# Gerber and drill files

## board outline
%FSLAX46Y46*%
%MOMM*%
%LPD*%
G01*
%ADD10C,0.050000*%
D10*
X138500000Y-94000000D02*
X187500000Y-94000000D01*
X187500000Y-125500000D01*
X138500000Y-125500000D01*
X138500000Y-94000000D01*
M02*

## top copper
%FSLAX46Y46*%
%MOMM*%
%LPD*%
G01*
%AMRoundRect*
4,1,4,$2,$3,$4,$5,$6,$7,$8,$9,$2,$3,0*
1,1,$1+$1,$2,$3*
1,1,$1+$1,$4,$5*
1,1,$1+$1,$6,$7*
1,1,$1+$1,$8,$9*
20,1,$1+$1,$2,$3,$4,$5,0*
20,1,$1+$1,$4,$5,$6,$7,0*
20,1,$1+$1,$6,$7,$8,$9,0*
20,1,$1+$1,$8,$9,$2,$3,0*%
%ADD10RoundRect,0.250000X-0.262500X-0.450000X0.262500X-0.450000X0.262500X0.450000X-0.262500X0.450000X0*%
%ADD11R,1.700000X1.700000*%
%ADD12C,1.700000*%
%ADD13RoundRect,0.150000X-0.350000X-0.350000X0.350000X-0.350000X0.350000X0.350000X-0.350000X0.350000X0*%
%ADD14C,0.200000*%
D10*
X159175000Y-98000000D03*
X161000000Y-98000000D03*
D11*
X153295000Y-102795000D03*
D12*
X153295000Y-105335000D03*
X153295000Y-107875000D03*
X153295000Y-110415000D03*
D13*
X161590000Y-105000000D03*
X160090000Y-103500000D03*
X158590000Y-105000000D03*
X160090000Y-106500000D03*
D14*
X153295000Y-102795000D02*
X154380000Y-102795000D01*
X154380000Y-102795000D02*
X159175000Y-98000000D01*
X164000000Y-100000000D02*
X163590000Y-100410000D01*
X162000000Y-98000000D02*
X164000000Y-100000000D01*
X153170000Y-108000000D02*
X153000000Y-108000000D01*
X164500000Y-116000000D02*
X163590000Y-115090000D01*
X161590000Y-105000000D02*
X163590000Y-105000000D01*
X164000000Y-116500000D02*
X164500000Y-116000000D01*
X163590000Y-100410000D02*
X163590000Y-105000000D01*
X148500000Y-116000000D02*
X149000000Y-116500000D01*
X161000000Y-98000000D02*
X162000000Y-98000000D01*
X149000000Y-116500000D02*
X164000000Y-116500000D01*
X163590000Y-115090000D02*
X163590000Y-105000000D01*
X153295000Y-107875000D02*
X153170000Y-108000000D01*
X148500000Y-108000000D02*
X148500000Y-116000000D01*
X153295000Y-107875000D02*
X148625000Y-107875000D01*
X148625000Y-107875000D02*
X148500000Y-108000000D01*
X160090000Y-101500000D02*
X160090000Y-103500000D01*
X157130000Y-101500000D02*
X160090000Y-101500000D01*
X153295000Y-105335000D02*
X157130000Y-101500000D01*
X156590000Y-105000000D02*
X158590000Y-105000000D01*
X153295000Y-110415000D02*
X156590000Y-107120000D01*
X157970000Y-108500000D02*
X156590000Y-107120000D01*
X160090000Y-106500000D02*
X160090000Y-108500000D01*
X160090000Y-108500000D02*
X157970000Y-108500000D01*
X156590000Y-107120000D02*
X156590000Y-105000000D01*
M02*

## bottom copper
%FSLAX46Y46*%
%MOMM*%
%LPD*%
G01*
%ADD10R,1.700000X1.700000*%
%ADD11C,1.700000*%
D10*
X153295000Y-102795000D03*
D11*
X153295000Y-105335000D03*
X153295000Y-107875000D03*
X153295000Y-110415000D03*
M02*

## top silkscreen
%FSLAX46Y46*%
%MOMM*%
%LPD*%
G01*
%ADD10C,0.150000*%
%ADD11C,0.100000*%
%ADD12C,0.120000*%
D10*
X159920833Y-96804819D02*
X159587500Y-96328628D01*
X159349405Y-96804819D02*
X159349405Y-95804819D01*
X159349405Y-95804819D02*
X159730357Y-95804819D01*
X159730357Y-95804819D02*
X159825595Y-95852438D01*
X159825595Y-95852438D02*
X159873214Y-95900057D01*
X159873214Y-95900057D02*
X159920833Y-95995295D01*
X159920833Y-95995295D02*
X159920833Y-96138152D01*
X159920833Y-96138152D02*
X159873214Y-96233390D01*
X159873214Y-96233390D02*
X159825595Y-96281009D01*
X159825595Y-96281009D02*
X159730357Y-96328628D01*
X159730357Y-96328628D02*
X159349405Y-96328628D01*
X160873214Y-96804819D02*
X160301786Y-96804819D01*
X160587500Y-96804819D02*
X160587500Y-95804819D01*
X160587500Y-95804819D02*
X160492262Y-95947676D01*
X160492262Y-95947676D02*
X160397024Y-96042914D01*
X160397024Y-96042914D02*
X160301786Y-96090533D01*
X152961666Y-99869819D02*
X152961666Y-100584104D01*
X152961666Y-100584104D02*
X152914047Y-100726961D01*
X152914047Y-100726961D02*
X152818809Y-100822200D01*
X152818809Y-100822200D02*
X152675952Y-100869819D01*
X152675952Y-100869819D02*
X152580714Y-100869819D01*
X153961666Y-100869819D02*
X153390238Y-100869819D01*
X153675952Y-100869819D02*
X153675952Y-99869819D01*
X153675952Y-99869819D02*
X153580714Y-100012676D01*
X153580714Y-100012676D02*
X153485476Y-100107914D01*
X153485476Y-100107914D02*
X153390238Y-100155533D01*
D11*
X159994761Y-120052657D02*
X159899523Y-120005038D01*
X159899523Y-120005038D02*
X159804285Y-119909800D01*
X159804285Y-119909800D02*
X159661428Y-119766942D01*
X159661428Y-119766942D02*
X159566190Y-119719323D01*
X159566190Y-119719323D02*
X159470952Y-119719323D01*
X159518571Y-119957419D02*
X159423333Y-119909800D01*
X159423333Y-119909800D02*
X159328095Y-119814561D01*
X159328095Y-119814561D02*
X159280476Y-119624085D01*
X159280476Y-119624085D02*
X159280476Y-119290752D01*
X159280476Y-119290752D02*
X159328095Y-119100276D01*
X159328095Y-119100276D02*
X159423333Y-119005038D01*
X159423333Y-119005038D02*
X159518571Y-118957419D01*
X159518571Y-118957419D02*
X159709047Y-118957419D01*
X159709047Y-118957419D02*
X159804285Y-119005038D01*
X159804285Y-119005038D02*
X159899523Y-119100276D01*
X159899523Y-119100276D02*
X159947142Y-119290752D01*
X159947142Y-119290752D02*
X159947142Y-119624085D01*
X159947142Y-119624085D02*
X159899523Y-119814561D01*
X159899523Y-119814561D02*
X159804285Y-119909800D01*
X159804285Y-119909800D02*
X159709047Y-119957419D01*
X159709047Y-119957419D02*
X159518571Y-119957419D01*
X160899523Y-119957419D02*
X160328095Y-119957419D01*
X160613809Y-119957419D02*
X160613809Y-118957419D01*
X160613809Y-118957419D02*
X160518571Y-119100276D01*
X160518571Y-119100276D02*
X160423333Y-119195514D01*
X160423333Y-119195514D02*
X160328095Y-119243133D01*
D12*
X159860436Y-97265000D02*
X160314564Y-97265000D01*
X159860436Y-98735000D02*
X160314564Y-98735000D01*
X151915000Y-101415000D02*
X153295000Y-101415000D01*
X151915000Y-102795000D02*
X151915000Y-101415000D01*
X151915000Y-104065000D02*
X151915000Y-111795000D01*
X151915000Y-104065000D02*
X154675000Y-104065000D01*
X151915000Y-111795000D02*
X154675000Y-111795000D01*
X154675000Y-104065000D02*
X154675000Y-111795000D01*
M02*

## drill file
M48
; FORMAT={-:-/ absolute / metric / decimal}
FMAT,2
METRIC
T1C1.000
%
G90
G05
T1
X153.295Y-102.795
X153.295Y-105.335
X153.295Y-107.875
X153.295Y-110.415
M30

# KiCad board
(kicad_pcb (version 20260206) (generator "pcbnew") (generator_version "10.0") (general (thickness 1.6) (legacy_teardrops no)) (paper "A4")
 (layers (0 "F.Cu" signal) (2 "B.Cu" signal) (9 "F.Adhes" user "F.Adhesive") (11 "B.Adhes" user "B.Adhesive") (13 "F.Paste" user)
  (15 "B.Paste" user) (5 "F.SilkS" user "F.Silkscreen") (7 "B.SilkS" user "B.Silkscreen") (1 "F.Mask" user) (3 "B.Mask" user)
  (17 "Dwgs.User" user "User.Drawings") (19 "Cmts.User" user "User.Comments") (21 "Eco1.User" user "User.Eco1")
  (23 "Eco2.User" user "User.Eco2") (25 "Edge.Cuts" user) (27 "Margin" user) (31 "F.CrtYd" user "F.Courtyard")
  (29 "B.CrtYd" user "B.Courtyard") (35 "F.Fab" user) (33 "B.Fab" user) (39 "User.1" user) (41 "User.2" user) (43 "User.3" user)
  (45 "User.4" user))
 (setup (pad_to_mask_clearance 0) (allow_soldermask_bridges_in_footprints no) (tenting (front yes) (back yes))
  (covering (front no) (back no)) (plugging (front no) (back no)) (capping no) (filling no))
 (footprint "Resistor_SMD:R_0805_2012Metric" (layer "F.Cu") (at 160.0875 98)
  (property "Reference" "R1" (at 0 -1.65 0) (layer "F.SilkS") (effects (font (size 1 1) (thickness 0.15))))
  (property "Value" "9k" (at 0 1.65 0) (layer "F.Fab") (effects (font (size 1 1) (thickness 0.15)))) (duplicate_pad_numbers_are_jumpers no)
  (fp_line (start -0.227064 -0.735) (end 0.227064 -0.735) (stroke (width 0.12) (type solid)) (layer "F.SilkS"))
  (fp_line (start -0.227064 0.735) (end 0.227064 0.735) (stroke (width 0.12) (type solid)) (layer "F.SilkS"))
  (pad "1" smd roundrect (at -0.9125 0) (size 1.025 1.4) (layers "F.Cu" "F.Mask" "F.Paste") (roundrect_rratio 0.243902) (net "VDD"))
  (pad "2" smd roundrect (at 0.9125 0) (size 1.025 1.4) (layers "F.Cu" "F.Mask" "F.Paste") (roundrect_rratio 0.243902) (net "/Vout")))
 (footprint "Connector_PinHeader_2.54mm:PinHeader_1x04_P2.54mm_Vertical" (layer "F.Cu") (at 153.295 102.795)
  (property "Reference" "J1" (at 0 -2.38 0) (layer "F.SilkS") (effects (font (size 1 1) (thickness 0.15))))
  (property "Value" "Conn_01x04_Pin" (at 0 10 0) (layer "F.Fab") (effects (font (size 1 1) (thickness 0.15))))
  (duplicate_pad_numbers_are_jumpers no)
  (fp_line (start -1.38 -1.38) (end 0 -1.38) (stroke (width 0.12) (type solid)) (layer "F.SilkS"))
  (fp_line (start -1.38 0) (end -1.38 -1.38) (stroke (width 0.12) (type solid)) (layer "F.SilkS"))
  (fp_line (start -1.38 1.27) (end -1.38 9) (stroke (width 0.12) (type solid)) (layer "F.SilkS"))
  (fp_line (start -1.38 1.27) (end 1.38 1.27) (stroke (width 0.12) (type solid)) (layer "F.SilkS"))
  (fp_line (start -1.38 9) (end 1.38 9) (stroke (width 0.12) (type solid)) (layer "F.SilkS"))
  (fp_line (start 1.38 1.27) (end 1.38 9) (stroke (width 0.12) (type solid)) (layer "F.SilkS"))
  (pad "1" thru_hole rect (at 0 0) (size 1.7 1.7) (drill 1) (layers "*.Cu" "*.Mask") (remove_unused_layers no) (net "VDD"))
  (pad "2" thru_hole circle (at 0 2.54) (size 1.7 1.7) (drill 1) (layers "*.Cu" "*.Mask") (remove_unused_layers no) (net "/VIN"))
  (pad "3" thru_hole circle (at 0 5.08) (size 1.7 1.7) (drill 1) (layers "*.Cu" "*.Mask") (remove_unused_layers no) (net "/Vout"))
  (pad "4" thru_hole circle (at 0 7.62) (size 1.7 1.7) (drill 1) (layers "*.Cu" "*.Mask") (remove_unused_layers no) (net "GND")))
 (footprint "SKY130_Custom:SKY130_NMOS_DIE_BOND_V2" (layer "F.Cu") (at 160.09 105)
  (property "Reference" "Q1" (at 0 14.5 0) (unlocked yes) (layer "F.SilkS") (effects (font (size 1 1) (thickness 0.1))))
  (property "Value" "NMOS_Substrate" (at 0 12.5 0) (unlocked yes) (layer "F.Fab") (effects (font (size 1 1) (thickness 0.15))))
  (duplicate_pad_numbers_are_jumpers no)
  (pad "1" smd roundrect (at 1.5 0) (size 1 1) (layers "F.Cu" "F.Mask") (roundrect_rratio 0.15) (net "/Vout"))
  (pad "2" smd roundrect (at 0 -1.5) (size 1 1) (layers "F.Cu" "F.Mask") (roundrect_rratio 0.15) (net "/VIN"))
  (pad "3" smd roundrect (at -1.5 0) (size 1 1) (layers "F.Cu" "F.Mask") (roundrect_rratio 0.15) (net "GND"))
  (pad "4" smd roundrect (at 0 1.5) (size 1 1) (layers "F.Cu" "F.Mask") (roundrect_rratio 0.15) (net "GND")))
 (gr_rect (start 138.5 94) (end 187.5 125.5) (stroke (width 0.05) (type default)) (fill no) (layer "Edge.Cuts"))
 (segment (start 153.295 102.795) (end 154.38 102.795) (width 0.2) (layer "F.Cu") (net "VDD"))
 (segment (start 154.38 102.795) (end 159.175 98) (width 0.2) (layer "F.Cu") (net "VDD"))
 (segment (start 164 100) (end 163.59 100.41) (width 0.2) (layer "F.Cu") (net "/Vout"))
 (segment (start 162 98) (end 164 100) (width 0.2) (layer "F.Cu") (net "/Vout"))
 (segment (start 153.17 108) (end 153 108) (width 0.2) (layer "F.Cu") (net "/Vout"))
 (segment (start 164.5 116) (end 163.59 115.09) (width 0.2) (layer "F.Cu") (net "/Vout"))
 (segment (start 161.59 105) (end 163.59 105) (width 0.2) (layer "F.Cu") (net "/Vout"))
 (segment (start 164 116.5) (end 164.5 116) (width 0.2) (layer "F.Cu") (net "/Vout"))
 (segment (start 163.59 100.41) (end 163.59 105) (width 0.2) (layer "F.Cu") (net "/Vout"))
 (segment (start 148.5 116) (end 149 116.5) (width 0.2) (layer "F.Cu") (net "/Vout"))
 (segment (start 161 98) (end 162 98) (width 0.2) (layer "F.Cu") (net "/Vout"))
 (segment (start 149 116.5) (end 164 116.5) (width 0.2) (layer "F.Cu") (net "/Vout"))
 (segment (start 163.59 115.09) (end 163.59 105) (width 0.2) (layer "F.Cu") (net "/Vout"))
 (segment (start 153.295 107.875) (end 153.17 108) (width 0.2) (layer "F.Cu") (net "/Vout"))
 (segment (start 148.5 108) (end 148.5 116) (width 0.2) (layer "F.Cu") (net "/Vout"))
 (segment (start 153.295 107.875) (end 148.625 107.875) (width 0.2) (layer "F.Cu") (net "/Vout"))
 (segment (start 148.625 107.875) (end 148.5 108) (width 0.2) (layer "F.Cu") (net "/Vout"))
 (segment (start 160.09 101.5) (end 160.09 103.5) (width 0.2) (layer "F.Cu") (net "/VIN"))
 (segment (start 157.13 101.5) (end 160.09 101.5) (width 0.2) (layer "F.Cu") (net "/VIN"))
 (segment (start 153.295 105.335) (end 157.13 101.5) (width 0.2) (layer "F.Cu") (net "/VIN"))
 (segment (start 156.59 105) (end 158.59 105) (width 0.2) (layer "F.Cu") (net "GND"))
 (segment (start 153.295 110.415) (end 156.59 107.12) (width 0.2) (layer "F.Cu") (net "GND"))
 (segment (start 157.97 108.5) (end 156.59 107.12) (width 0.2) (layer "F.Cu") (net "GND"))
 (segment (start 160.09 106.5) (end 160.09 108.5) (width 0.2) (layer "F.Cu") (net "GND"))
 (segment (start 160.09 108.5) (end 157.97 108.5) (width 0.2) (layer "F.Cu") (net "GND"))
 (segment (start 156.59 107.12) (end 156.59 105) (width 0.2) (layer "F.Cu") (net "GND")))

